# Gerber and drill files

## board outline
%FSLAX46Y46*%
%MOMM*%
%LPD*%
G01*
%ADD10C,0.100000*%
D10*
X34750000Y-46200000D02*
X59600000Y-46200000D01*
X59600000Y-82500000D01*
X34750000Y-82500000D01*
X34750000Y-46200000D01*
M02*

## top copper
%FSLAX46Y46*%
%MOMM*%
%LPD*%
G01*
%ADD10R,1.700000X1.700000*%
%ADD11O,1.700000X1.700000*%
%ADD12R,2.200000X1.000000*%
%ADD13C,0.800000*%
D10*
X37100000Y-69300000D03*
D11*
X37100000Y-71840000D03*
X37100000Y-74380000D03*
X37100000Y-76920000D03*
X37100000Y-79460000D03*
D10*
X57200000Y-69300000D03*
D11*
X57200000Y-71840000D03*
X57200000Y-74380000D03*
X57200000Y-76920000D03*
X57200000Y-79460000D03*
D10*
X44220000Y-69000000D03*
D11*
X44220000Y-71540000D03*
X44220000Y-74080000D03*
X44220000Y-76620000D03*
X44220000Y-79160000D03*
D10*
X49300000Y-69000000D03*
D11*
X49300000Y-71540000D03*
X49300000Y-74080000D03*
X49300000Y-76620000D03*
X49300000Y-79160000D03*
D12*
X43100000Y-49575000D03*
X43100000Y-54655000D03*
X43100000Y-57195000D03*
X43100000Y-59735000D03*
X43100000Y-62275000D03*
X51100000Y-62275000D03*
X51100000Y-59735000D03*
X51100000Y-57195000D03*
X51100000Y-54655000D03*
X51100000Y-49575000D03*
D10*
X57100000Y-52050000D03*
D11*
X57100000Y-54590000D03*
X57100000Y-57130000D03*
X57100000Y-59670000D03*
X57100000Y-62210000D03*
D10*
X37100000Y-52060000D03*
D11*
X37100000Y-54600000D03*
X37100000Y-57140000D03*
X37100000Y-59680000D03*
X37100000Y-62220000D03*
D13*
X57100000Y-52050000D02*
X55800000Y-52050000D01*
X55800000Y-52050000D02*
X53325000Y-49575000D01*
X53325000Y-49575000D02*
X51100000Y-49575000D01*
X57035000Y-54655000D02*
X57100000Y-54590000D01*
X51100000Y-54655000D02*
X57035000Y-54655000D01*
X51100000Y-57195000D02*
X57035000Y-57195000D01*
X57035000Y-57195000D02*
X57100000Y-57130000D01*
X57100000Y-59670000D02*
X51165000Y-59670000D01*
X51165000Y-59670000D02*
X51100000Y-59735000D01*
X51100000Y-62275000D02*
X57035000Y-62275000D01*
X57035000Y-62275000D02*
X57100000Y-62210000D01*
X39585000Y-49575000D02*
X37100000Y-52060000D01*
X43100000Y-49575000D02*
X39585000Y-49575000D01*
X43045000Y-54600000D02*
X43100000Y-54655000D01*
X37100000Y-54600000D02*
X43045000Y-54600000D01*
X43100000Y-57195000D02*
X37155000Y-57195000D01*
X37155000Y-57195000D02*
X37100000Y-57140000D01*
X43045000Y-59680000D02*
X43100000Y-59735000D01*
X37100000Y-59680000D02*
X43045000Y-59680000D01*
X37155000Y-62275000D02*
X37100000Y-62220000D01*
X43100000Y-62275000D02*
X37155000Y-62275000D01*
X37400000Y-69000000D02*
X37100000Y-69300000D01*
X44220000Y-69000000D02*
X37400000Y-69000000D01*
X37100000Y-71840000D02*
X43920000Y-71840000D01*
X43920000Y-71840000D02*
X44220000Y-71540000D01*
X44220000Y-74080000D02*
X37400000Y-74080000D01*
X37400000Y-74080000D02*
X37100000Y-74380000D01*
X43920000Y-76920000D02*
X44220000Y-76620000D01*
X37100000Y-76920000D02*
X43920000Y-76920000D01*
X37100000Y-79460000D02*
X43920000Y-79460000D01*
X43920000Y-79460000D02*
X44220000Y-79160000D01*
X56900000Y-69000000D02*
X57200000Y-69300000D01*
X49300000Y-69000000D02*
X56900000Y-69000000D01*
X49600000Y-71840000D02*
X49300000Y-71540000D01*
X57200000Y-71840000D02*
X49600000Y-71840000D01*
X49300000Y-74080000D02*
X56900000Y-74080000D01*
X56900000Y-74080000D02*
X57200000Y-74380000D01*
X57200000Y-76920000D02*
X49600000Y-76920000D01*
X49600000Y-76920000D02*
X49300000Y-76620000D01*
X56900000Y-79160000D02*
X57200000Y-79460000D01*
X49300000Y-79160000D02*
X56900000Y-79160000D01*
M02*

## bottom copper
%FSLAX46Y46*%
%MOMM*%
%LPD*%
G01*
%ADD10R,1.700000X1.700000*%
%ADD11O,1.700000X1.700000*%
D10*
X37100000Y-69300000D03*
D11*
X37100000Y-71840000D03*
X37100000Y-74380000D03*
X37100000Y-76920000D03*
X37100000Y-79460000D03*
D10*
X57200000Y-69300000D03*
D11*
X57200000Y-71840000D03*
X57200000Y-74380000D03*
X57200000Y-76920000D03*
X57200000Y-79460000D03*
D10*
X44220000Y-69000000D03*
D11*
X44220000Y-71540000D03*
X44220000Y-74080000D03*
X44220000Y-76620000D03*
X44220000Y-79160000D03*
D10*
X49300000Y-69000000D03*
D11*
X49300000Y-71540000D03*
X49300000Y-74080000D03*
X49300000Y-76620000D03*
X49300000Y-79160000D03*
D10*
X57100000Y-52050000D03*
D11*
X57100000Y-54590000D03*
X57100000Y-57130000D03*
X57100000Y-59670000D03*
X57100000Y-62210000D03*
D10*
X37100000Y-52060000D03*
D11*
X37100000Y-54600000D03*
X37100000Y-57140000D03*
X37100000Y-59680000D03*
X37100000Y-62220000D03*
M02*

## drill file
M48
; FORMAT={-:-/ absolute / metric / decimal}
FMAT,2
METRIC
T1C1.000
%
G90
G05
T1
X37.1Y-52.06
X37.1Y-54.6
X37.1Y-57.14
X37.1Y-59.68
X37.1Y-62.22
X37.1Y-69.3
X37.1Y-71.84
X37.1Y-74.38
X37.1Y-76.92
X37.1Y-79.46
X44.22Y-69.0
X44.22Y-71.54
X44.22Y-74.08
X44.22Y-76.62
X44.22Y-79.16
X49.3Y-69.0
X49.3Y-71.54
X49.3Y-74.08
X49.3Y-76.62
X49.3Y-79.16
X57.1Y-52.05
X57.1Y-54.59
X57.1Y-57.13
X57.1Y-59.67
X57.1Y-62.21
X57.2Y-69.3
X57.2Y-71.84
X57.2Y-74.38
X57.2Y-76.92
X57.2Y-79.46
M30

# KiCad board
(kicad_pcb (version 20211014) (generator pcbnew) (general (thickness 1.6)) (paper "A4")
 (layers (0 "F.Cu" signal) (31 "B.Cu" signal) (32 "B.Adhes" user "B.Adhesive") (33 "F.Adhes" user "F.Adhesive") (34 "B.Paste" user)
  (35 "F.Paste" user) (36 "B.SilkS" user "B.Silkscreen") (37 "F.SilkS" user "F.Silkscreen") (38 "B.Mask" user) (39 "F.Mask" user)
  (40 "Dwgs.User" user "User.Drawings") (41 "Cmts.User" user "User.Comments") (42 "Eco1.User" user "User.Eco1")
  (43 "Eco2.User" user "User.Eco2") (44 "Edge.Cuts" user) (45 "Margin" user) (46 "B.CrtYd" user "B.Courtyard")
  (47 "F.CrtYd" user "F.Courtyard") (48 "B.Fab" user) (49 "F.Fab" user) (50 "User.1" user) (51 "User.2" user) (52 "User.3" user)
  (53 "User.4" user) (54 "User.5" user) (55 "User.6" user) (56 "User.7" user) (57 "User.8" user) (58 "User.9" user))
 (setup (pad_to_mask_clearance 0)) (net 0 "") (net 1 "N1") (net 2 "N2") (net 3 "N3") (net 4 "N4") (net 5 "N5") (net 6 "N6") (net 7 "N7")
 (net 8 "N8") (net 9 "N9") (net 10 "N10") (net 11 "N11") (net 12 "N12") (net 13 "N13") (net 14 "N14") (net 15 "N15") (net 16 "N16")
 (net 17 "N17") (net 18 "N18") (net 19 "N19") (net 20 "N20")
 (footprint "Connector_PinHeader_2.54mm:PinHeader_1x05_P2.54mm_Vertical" (layer "F.Cu") (at 37.1 69.3)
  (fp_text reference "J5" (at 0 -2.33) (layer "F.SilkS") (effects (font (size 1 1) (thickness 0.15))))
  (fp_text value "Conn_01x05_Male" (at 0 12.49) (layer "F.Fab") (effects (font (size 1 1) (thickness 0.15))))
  (pad "1" thru_hole rect (at 0 0) (size 1.7 1.7) (drill 1) (layers *.Cu *.Mask) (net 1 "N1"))
  (pad "2" thru_hole oval (at 0 2.54) (size 1.7 1.7) (drill 1) (layers *.Cu *.Mask) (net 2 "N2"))
  (pad "3" thru_hole oval (at 0 5.08) (size 1.7 1.7) (drill 1) (layers *.Cu *.Mask) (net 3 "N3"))
  (pad "4" thru_hole oval (at 0 7.62) (size 1.7 1.7) (drill 1) (layers *.Cu *.Mask) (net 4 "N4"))
  (pad "5" thru_hole oval (at 0 10.16) (size 1.7 1.7) (drill 1) (layers *.Cu *.Mask) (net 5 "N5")))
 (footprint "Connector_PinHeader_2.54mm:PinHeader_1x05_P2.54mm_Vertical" (layer "F.Cu") (at 57.2 69.3)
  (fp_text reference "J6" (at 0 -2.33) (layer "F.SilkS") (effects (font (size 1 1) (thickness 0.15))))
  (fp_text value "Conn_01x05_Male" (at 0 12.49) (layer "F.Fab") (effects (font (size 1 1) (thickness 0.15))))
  (pad "1" thru_hole rect (at 0 0) (size 1.7 1.7) (drill 1) (layers *.Cu *.Mask) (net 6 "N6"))
  (pad "2" thru_hole oval (at 0 2.54) (size 1.7 1.7) (drill 1) (layers *.Cu *.Mask) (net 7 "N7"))
  (pad "3" thru_hole oval (at 0 5.08) (size 1.7 1.7) (drill 1) (layers *.Cu *.Mask) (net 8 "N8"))
  (pad "4" thru_hole oval (at 0 7.62) (size 1.7 1.7) (drill 1) (layers *.Cu *.Mask) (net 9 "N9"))
  (pad "5" thru_hole oval (at 0 10.16) (size 1.7 1.7) (drill 1) (layers *.Cu *.Mask) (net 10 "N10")))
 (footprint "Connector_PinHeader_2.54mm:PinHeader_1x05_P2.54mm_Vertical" (layer "F.Cu") (at 44.22 69)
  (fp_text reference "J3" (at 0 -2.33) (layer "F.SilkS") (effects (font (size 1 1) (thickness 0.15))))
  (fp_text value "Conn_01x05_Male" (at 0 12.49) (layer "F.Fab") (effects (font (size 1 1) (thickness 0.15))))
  (pad "1" thru_hole rect (at 0 0) (size 1.7 1.7) (drill 1) (layers *.Cu *.Mask) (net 1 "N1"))
  (pad "2" thru_hole oval (at 0 2.54) (size 1.7 1.7) (drill 1) (layers *.Cu *.Mask) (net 2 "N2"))
  (pad "3" thru_hole oval (at 0 5.08) (size 1.7 1.7) (drill 1) (layers *.Cu *.Mask) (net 3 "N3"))
  (pad "4" thru_hole oval (at 0 7.62) (size 1.7 1.7) (drill 1) (layers *.Cu *.Mask) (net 4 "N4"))
  (pad "5" thru_hole oval (at 0 10.16) (size 1.7 1.7) (drill 1) (layers *.Cu *.Mask) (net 5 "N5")))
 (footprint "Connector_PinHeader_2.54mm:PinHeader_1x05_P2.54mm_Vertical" (layer "F.Cu") (at 49.3 69)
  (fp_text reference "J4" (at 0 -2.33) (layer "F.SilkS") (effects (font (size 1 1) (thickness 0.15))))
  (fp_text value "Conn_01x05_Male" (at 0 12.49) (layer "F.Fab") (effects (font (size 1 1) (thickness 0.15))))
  (pad "1" thru_hole rect (at 0 0) (size 1.7 1.7) (drill 1) (layers *.Cu *.Mask) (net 6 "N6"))
  (pad "2" thru_hole oval (at 0 2.54) (size 1.7 1.7) (drill 1) (layers *.Cu *.Mask) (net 7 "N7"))
  (pad "3" thru_hole oval (at 0 5.08) (size 1.7 1.7) (drill 1) (layers *.Cu *.Mask) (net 8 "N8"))
  (pad "4" thru_hole oval (at 0 7.62) (size 1.7 1.7) (drill 1) (layers *.Cu *.Mask) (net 9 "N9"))
  (pad "5" thru_hole oval (at 0 10.16) (size 1.7 1.7) (drill 1) (layers *.Cu *.Mask) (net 10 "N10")))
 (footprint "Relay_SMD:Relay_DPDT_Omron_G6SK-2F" (layer "F.Cu") (at 47.1 55.925)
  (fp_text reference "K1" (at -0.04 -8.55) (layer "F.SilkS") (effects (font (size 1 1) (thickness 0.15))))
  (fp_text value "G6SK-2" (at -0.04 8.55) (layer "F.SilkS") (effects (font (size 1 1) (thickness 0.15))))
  (pad "1" smd rect (at -4 -6.35) (size 2.2 1) (layers "F.Cu" "F.Paste" "F.Mask") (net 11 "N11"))
  (pad "3" smd rect (at -4 -1.27) (size 2.2 1) (layers "F.Cu" "F.Paste" "F.Mask") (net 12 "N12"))
  (pad "4" smd rect (at -4 1.27) (size 2.2 1) (layers "F.Cu" "F.Paste" "F.Mask") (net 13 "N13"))
  (pad "5" smd rect (at -4 3.81) (size 2.2 1) (layers "F.Cu" "F.Paste" "F.Mask") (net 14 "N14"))
  (pad "6" smd rect (at -4 6.35) (size 2.2 1) (layers "F.Cu" "F.Paste" "F.Mask") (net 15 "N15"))
  (pad "7" smd rect (at 4 6.35) (size 2.2 1) (layers "F.Cu" "F.Paste" "F.Mask") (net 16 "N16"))
  (pad "8" smd rect (at 4 3.81) (size 2.2 1) (layers "F.Cu" "F.Paste" "F.Mask") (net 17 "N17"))
  (pad "9" smd rect (at 4 1.27) (size 2.2 1) (layers "F.Cu" "F.Paste" "F.Mask") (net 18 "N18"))
  (pad "10" smd rect (at 4 -1.27) (size 2.2 1) (layers "F.Cu" "F.Paste" "F.Mask") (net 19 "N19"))
  (pad "12" smd rect (at 4 -6.35) (size 2.2 1) (layers "F.Cu" "F.Paste" "F.Mask") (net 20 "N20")))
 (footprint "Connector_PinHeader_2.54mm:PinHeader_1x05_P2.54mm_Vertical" (layer "F.Cu") (at 57.1 52.05)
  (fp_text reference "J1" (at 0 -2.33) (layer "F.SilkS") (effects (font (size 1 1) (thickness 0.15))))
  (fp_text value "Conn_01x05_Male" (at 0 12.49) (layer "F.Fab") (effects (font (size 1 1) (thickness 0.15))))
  (pad "1" thru_hole rect (at 0 0) (size 1.7 1.7) (drill 1) (layers *.Cu *.Mask) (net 20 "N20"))
  (pad "2" thru_hole oval (at 0 2.54) (size 1.7 1.7) (drill 1) (layers *.Cu *.Mask) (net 19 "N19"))
  (pad "3" thru_hole oval (at 0 5.08) (size 1.7 1.7) (drill 1) (layers *.Cu *.Mask) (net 18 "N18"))
  (pad "4" thru_hole oval (at 0 7.62) (size 1.7 1.7) (drill 1) (layers *.Cu *.Mask) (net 17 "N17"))
  (pad "5" thru_hole oval (at 0 10.16) (size 1.7 1.7) (drill 1) (layers *.Cu *.Mask) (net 16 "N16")))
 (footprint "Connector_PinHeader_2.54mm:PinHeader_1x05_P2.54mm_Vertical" (layer "F.Cu") (at 37.1 52.06)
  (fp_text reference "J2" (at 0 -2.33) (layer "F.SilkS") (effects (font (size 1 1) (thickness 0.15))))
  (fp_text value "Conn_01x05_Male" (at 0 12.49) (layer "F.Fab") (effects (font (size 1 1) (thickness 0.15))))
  (pad "1" thru_hole rect (at 0 0) (size 1.7 1.7) (drill 1) (layers *.Cu *.Mask) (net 11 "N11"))
  (pad "2" thru_hole oval (at 0 2.54) (size 1.7 1.7) (drill 1) (layers *.Cu *.Mask) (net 12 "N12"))
  (pad "3" thru_hole oval (at 0 5.08) (size 1.7 1.7) (drill 1) (layers *.Cu *.Mask) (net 13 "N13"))
  (pad "4" thru_hole oval (at 0 7.62) (size 1.7 1.7) (drill 1) (layers *.Cu *.Mask) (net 14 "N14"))
  (pad "5" thru_hole oval (at 0 10.16) (size 1.7 1.7) (drill 1) (layers *.Cu *.Mask) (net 15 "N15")))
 (gr_rect (start 34.75 46.2) (end 59.6 82.5) (layer "Edge.Cuts") (width 0.1) (fill none))
 (segment (start 57.1 52.05) (end 55.8 52.05) (width 0.8) (layer "F.Cu") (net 20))
 (segment (start 55.8 52.05) (end 53.325 49.575) (width 0.8) (layer "F.Cu") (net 20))
 (segment (start 53.325 49.575) (end 51.1 49.575) (width 0.8) (layer "F.Cu") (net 20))
 (segment (start 57.035 54.655) (end 57.1 54.59) (width 0.8) (layer "F.Cu") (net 19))
 (segment (start 51.1 54.655) (end 57.035 54.655) (width 0.8) (layer "F.Cu") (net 19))
 (segment (start 51.1 57.195) (end 57.035 57.195) (width 0.8) (layer "F.Cu") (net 18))
 (segment (start 57.035 57.195) (end 57.1 57.13) (width 0.8) (layer "F.Cu") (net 18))
 (segment (start 57.1 59.67) (end 51.165 59.67) (width 0.8) (layer "F.Cu") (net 17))
 (segment (start 51.165 59.67) (end 51.1 59.735) (width 0.8) (layer "F.Cu") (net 17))
 (segment (start 51.1 62.275) (end 57.035 62.275) (width 0.8) (layer "F.Cu") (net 16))
 (segment (start 57.035 62.275) (end 57.1 62.21) (width 0.8) (layer "F.Cu") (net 16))
 (segment (start 39.585 49.575) (end 37.1 52.06) (width 0.8) (layer "F.Cu") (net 11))
 (segment (start 43.1 49.575) (end 39.585 49.575) (width 0.8) (layer "F.Cu") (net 11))
 (segment (start 43.045 54.6) (end 43.1 54.655) (width 0.8) (layer "F.Cu") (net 12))
 (segment (start 37.1 54.6) (end 43.045 54.6) (width 0.8) (layer "F.Cu") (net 12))
 (segment (start 43.1 57.195) (end 37.155 57.195) (width 0.8) (layer "F.Cu") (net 13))
 (segment (start 37.155 57.195) (end 37.1 57.14) (width 0.8) (layer "F.Cu") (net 13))
 (segment (start 43.045 59.68) (end 43.1 59.735) (width 0.8) (layer "F.Cu") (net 14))
 (segment (start 37.1 59.68) (end 43.045 59.68) (width 0.8) (layer "F.Cu") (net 14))
 (segment (start 37.155 62.275) (end 37.1 62.22) (width 0.8) (layer "F.Cu") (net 15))
 (segment (start 43.1 62.275) (end 37.155 62.275) (width 0.8) (layer "F.Cu") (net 15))
 (segment (start 37.4 69) (end 37.1 69.3) (width 0.8) (layer "F.Cu") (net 1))
 (segment (start 44.22 69) (end 37.4 69) (width 0.8) (layer "F.Cu") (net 1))
 (segment (start 37.1 71.84) (end 43.92 71.84) (width 0.8) (layer "F.Cu") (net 2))
 (segment (start 43.92 71.84) (end 44.22 71.54) (width 0.8) (layer "F.Cu") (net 2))
 (segment (start 44.22 74.08) (end 37.4 74.08) (width 0.8) (layer "F.Cu") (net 3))
 (segment (start 37.4 74.08) (end 37.1 74.38) (width 0.8) (layer "F.Cu") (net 3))
 (segment (start 43.92 76.92) (end 44.22 76.62) (width 0.8) (layer "F.Cu") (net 4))
 (segment (start 37.1 76.92) (end 43.92 76.92) (width 0.8) (layer "F.Cu") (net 4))
 (segment (start 37.1 79.46) (end 43.92 79.46) (width 0.8) (layer "F.Cu") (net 5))
 (segment (start 43.92 79.46) (end 44.22 79.16) (width 0.8) (layer "F.Cu") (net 5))
 (segment (start 56.9 69) (end 57.2 69.3) (width 0.8) (layer "F.Cu") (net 6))
 (segment (start 49.3 69) (end 56.9 69) (width 0.8) (layer "F.Cu") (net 6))
 (segment (start 49.6 71.84) (end 49.3 71.54) (width 0.8) (layer "F.Cu") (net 7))
 (segment (start 57.2 71.84) (end 49.6 71.84) (width 0.8) (layer "F.Cu") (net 7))
 (segment (start 49.3 74.08) (end 56.9 74.08) (width 0.8) (layer "F.Cu") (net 8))
 (segment (start 56.9 74.08) (end 57.2 74.38) (width 0.8) (layer "F.Cu") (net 8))
 (segment (start 57.2 76.92) (end 49.6 76.92) (width 0.8) (layer "F.Cu") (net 9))
 (segment (start 49.6 76.92) (end 49.3 76.62) (width 0.8) (layer "F.Cu") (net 9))
 (segment (start 56.9 79.16) (end 57.2 79.46) (width 0.8) (layer "F.Cu") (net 10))
 (segment (start 49.3 79.16) (end 56.9 79.16) (width 0.8) (layer "F.Cu") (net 10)))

